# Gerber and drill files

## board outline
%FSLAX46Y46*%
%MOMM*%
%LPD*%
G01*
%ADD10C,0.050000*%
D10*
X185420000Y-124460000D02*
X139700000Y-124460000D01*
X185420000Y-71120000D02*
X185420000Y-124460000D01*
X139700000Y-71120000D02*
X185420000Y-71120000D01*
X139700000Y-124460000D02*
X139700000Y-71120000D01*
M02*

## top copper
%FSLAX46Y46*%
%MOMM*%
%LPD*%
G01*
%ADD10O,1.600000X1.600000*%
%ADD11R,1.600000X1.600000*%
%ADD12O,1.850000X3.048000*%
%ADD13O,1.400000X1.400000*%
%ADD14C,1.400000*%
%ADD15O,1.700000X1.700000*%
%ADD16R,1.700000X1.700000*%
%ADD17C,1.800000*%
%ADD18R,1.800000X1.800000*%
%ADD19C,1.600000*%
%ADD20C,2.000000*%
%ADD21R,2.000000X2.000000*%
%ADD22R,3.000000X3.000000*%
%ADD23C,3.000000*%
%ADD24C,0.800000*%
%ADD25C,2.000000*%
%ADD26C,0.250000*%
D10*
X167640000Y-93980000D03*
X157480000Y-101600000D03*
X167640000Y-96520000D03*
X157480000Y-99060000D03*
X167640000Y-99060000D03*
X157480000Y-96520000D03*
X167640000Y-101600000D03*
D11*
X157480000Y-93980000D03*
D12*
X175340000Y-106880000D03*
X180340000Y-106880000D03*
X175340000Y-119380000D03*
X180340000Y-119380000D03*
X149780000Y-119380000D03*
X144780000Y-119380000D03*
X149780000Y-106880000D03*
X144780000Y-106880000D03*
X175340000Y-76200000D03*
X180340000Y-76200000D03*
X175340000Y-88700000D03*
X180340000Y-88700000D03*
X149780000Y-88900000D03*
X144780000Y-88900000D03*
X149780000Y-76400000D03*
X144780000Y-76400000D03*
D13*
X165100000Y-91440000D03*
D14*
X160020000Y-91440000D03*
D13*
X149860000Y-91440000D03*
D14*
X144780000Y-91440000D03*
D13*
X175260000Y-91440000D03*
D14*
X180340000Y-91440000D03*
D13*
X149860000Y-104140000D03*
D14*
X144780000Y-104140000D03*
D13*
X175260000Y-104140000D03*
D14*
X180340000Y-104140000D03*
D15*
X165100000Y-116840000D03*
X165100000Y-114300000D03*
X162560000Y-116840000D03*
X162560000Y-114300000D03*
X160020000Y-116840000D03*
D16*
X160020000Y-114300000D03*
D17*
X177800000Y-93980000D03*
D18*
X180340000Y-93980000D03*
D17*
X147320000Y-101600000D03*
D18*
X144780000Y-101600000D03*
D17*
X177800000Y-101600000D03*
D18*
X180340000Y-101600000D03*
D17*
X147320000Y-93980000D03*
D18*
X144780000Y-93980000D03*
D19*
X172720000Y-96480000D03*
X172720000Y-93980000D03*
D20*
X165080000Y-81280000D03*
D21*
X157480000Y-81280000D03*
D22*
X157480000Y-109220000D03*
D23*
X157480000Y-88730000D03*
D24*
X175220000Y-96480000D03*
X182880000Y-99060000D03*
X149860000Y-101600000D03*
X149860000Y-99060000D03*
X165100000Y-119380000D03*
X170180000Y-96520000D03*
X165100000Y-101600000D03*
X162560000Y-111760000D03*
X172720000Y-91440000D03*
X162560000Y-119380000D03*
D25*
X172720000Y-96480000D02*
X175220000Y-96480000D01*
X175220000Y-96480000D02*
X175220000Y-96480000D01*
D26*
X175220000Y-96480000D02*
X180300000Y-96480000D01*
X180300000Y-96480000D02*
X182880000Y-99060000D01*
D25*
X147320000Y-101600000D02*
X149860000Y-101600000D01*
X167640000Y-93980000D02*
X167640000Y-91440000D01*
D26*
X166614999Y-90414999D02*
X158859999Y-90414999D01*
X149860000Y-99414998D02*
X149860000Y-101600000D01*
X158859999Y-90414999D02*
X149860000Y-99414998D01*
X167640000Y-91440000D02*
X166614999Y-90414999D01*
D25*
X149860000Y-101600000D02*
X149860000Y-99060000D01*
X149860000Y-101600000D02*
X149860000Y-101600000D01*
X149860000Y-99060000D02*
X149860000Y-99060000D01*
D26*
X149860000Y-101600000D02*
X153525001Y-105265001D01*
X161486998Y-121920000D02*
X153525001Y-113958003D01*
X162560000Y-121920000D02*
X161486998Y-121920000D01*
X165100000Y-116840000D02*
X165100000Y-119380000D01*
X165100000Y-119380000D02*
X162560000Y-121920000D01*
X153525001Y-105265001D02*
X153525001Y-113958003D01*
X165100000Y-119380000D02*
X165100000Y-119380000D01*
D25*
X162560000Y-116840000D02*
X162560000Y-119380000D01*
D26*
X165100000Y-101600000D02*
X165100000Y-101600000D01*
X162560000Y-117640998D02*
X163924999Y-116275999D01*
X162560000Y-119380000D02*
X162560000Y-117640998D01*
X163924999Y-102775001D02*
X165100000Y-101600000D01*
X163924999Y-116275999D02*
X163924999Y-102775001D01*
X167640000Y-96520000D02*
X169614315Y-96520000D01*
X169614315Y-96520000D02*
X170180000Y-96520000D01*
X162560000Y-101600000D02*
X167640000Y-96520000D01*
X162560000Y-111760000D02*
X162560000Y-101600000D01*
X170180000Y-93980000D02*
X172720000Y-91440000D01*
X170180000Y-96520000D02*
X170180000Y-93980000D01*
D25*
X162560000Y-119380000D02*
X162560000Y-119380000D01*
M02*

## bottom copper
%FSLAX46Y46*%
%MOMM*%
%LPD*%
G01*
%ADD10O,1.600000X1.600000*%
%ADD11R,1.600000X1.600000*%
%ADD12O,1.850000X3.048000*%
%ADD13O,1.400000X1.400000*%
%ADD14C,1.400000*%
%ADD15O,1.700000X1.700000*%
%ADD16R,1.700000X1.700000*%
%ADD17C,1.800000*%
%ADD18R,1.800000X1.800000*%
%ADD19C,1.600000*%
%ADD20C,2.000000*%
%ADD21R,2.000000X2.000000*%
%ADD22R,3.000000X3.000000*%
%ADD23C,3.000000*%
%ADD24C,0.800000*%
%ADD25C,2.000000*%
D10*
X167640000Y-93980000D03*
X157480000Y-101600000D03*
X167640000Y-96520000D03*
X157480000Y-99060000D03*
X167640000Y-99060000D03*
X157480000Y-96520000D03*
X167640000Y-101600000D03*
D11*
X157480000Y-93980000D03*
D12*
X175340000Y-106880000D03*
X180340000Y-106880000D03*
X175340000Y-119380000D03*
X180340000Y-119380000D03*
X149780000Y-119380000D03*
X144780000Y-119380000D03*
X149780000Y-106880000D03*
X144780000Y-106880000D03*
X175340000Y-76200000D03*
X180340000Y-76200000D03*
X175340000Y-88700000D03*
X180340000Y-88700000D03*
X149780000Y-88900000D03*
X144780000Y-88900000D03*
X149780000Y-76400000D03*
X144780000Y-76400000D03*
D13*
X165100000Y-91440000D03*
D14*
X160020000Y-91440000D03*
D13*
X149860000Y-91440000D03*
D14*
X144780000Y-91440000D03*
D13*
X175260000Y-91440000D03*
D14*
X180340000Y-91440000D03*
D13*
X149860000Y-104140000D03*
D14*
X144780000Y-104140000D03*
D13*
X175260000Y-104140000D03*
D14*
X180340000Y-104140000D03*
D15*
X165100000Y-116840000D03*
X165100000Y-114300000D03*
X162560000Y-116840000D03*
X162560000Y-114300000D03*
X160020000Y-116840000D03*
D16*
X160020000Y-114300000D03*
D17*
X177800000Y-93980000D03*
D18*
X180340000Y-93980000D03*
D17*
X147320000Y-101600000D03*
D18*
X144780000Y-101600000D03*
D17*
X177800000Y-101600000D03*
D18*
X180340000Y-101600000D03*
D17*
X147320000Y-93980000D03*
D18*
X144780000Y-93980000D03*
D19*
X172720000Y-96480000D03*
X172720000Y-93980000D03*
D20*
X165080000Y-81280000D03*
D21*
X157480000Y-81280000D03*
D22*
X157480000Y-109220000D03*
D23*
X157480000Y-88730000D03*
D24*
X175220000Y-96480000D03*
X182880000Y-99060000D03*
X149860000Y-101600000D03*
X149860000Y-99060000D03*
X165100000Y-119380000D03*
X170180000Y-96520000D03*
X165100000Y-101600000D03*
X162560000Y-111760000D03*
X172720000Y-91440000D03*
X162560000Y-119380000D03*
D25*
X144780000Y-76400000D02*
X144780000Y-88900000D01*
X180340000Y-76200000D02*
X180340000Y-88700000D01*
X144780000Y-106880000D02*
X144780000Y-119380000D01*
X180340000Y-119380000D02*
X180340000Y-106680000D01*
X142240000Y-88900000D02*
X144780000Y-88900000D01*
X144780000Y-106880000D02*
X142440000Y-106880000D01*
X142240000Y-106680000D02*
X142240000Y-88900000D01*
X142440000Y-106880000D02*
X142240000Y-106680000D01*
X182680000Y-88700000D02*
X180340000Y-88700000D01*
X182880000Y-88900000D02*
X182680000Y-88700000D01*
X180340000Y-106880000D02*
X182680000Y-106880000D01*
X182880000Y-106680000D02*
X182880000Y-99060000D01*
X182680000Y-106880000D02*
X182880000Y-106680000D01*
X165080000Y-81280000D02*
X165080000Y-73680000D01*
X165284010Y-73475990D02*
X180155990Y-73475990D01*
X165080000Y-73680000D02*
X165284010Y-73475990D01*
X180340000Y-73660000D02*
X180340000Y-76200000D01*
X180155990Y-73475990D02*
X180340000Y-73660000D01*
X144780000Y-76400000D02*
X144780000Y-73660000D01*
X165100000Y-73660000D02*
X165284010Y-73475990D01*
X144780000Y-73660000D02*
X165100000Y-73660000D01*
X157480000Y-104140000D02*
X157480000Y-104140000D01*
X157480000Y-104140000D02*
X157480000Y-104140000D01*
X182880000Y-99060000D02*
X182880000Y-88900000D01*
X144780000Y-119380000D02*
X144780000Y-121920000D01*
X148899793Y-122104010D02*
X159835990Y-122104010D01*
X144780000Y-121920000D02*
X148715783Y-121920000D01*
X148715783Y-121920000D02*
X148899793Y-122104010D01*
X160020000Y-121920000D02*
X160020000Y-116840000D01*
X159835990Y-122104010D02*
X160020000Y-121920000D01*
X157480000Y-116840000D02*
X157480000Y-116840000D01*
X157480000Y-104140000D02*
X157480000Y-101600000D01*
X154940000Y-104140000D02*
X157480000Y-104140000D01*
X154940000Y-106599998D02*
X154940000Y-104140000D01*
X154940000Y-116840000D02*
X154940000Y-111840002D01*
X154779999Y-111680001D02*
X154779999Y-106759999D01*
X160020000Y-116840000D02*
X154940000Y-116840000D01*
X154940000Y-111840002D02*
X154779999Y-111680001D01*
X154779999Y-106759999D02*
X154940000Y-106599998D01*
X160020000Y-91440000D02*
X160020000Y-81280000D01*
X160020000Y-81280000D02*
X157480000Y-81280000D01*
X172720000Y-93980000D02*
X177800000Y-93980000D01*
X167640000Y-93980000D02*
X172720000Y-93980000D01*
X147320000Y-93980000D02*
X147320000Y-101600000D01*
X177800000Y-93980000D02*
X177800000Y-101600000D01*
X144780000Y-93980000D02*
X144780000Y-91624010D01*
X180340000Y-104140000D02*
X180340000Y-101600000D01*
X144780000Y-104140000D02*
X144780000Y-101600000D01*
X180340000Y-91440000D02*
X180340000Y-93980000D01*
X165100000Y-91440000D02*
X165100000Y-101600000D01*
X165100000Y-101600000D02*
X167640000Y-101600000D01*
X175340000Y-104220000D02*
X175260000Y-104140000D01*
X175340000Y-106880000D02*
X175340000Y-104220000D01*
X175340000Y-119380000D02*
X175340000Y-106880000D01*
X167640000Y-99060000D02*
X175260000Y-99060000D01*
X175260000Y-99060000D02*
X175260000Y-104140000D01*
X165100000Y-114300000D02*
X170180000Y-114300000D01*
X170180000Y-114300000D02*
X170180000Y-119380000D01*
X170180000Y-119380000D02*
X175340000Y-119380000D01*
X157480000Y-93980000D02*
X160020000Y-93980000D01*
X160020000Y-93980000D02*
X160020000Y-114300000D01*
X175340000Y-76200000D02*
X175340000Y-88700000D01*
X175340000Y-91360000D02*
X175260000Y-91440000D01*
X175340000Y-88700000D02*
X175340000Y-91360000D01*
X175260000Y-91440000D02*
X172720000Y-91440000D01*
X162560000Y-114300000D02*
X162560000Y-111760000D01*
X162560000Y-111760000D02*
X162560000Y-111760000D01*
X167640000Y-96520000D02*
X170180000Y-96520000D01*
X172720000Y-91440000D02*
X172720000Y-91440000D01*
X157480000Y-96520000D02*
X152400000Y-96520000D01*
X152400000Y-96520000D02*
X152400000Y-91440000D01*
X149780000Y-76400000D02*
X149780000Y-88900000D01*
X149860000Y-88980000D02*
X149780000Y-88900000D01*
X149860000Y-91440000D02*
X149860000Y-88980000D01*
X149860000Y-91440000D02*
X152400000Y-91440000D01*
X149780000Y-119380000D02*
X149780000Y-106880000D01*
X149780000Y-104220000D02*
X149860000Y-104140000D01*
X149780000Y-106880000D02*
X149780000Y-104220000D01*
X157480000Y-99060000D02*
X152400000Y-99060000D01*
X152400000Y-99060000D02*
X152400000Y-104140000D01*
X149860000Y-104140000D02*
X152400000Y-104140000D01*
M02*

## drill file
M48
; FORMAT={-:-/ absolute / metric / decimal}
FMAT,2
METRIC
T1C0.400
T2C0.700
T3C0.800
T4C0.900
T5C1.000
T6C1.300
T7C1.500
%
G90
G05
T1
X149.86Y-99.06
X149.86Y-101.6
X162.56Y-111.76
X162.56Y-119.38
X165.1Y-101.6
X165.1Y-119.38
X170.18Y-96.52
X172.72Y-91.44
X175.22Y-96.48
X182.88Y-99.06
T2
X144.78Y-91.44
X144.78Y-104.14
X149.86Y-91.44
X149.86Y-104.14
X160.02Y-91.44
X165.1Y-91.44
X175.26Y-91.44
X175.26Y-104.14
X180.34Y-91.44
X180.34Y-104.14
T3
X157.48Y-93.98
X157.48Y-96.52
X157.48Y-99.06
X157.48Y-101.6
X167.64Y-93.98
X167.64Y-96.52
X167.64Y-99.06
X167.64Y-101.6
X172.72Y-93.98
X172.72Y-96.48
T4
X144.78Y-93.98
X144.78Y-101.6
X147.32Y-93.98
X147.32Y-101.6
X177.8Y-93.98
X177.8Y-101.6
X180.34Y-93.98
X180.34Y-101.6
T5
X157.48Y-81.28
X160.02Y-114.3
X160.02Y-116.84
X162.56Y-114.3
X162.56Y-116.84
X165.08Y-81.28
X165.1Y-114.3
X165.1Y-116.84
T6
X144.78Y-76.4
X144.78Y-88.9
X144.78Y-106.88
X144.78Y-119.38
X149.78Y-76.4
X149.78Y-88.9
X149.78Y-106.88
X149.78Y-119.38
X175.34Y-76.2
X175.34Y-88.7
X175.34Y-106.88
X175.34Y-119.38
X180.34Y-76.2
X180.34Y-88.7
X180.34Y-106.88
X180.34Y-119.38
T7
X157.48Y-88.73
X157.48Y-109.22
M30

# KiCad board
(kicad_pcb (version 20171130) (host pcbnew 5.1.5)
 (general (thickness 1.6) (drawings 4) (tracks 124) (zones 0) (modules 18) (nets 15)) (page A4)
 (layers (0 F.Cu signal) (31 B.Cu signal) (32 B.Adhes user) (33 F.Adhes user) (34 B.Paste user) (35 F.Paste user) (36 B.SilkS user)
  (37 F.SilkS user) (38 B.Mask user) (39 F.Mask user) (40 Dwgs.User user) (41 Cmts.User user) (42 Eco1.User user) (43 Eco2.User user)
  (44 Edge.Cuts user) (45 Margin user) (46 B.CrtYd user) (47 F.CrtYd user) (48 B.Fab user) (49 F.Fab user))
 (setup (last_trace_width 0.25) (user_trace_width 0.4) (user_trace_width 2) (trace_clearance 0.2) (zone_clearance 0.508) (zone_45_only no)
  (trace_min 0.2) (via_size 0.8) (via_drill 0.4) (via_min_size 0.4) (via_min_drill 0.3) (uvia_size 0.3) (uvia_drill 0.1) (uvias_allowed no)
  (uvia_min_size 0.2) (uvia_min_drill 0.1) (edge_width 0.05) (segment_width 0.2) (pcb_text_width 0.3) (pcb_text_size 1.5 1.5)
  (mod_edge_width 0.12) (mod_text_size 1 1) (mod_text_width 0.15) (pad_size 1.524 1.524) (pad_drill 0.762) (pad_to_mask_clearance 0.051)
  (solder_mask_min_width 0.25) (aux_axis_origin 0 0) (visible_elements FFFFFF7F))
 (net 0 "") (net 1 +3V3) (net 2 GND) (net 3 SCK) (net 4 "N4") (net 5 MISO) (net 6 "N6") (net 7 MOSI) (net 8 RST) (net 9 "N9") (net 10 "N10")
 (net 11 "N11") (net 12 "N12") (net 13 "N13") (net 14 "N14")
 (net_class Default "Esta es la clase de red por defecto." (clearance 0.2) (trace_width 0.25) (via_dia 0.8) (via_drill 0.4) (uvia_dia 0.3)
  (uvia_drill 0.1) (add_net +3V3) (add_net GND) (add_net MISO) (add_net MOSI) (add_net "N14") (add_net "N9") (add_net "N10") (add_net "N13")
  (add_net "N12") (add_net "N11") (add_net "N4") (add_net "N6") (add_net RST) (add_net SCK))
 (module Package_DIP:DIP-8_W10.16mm (layer F.Cu) (at 157.48 93.98)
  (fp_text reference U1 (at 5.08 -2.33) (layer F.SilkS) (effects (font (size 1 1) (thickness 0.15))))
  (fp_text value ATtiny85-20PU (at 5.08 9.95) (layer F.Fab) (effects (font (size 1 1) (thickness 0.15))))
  (pad 8 thru_hole oval (at 10.16 0) (size 1.6 1.6) (drill 0.8) (layers *.Cu *.Mask) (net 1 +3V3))
  (pad 4 thru_hole oval (at 0 7.62) (size 1.6 1.6) (drill 0.8) (layers *.Cu *.Mask) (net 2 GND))
  (pad 7 thru_hole oval (at 10.16 2.54) (size 1.6 1.6) (drill 0.8) (layers *.Cu *.Mask) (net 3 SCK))
  (pad 3 thru_hole oval (at 0 5.08) (size 1.6 1.6) (drill 0.8) (layers *.Cu *.Mask) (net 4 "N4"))
  (pad 6 thru_hole oval (at 10.16 5.08) (size 1.6 1.6) (drill 0.8) (layers *.Cu *.Mask) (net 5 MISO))
  (pad 2 thru_hole oval (at 0 2.54) (size 1.6 1.6) (drill 0.8) (layers *.Cu *.Mask) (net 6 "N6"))
  (pad 5 thru_hole oval (at 10.16 7.62) (size 1.6 1.6) (drill 0.8) (layers *.Cu *.Mask) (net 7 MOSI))
  (pad 1 thru_hole rect (at 0 0) (size 1.6 1.6) (drill 0.8) (layers *.Cu *.Mask) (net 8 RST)))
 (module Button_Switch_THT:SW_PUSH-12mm (layer F.Cu) (at 180.34 106.88 270)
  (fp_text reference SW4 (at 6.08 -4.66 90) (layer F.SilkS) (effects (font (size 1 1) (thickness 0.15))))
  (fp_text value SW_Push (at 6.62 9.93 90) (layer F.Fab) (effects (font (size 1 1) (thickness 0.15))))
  (pad 2 thru_hole oval (at 0 5 270) (size 3.048 1.85) (drill 1.3) (layers *.Cu *.Mask) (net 5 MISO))
  (pad 1 thru_hole oval (at 0 0 270) (size 3.048 1.85) (drill 1.3) (layers *.Cu *.Mask) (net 2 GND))
  (pad 2 thru_hole oval (at 12.5 5 270) (size 3.048 1.85) (drill 1.3) (layers *.Cu *.Mask) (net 5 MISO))
  (pad 1 thru_hole oval (at 12.5 0 270) (size 3.048 1.85) (drill 1.3) (layers *.Cu *.Mask) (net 2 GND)))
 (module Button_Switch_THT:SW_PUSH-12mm (layer F.Cu) (at 144.78 119.38 90)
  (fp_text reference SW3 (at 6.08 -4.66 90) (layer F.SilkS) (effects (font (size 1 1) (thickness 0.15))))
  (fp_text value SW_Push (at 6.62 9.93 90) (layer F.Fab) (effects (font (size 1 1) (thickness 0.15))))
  (pad 2 thru_hole oval (at 0 5 90) (size 3.048 1.85) (drill 1.3) (layers *.Cu *.Mask) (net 4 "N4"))
  (pad 1 thru_hole oval (at 0 0 90) (size 3.048 1.85) (drill 1.3) (layers *.Cu *.Mask) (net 2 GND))
  (pad 2 thru_hole oval (at 12.5 5 90) (size 3.048 1.85) (drill 1.3) (layers *.Cu *.Mask) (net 4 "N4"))
  (pad 1 thru_hole oval (at 12.5 0 90) (size 3.048 1.85) (drill 1.3) (layers *.Cu *.Mask) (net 2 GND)))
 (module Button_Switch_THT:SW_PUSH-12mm (layer F.Cu) (at 180.34 76.2 270)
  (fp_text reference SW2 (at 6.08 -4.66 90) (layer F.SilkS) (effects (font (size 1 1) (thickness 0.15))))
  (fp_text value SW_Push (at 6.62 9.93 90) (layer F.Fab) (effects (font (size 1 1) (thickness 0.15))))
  (pad 2 thru_hole oval (at 0 5 270) (size 3.048 1.85) (drill 1.3) (layers *.Cu *.Mask) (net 3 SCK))
  (pad 1 thru_hole oval (at 0 0 270) (size 3.048 1.85) (drill 1.3) (layers *.Cu *.Mask) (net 2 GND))
  (pad 2 thru_hole oval (at 12.5 5 270) (size 3.048 1.85) (drill 1.3) (layers *.Cu *.Mask) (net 3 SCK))
  (pad 1 thru_hole oval (at 12.5 0 270) (size 3.048 1.85) (drill 1.3) (layers *.Cu *.Mask) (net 2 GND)))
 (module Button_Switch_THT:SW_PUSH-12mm (layer F.Cu) (at 144.78 88.9 90)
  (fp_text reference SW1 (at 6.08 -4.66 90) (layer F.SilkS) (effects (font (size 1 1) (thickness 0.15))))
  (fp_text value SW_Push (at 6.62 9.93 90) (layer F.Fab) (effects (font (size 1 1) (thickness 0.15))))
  (pad 2 thru_hole oval (at 0 5 90) (size 3.048 1.85) (drill 1.3) (layers *.Cu *.Mask) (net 6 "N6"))
  (pad 1 thru_hole oval (at 0 0 90) (size 3.048 1.85) (drill 1.3) (layers *.Cu *.Mask) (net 2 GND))
  (pad 2 thru_hole oval (at 12.5 5 90) (size 3.048 1.85) (drill 1.3) (layers *.Cu *.Mask) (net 6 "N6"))
  (pad 1 thru_hole oval (at 12.5 0 90) (size 3.048 1.85) (drill 1.3) (layers *.Cu *.Mask) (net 2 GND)))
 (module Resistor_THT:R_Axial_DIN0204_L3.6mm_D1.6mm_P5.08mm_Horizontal (layer F.Cu) (at 160.02 91.44)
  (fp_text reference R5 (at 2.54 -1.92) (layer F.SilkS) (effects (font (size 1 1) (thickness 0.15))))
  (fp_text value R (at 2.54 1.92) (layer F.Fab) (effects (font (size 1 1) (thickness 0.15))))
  (pad 2 thru_hole oval (at 5.08 0) (size 1.4 1.4) (drill 0.7) (layers *.Cu *.Mask) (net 7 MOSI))
  (pad 1 thru_hole circle (at 0 0) (size 1.4 1.4) (drill 0.7) (layers *.Cu *.Mask) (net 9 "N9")))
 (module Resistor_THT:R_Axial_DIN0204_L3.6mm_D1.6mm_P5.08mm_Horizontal (layer F.Cu) (at 144.78 91.44)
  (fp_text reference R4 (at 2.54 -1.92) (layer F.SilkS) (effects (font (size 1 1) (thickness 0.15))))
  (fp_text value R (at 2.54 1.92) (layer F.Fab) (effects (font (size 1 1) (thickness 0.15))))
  (pad 2 thru_hole oval (at 5.08 0) (size 1.4 1.4) (drill 0.7) (layers *.Cu *.Mask) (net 6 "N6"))
  (pad 1 thru_hole circle (at 0 0) (size 1.4 1.4) (drill 0.7) (layers *.Cu *.Mask) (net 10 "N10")))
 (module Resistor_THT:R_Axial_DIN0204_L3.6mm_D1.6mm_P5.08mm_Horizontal (layer F.Cu) (at 180.34 91.44 180)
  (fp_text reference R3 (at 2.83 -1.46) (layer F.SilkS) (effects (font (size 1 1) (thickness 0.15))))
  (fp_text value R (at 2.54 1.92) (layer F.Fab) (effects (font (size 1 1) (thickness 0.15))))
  (pad 2 thru_hole oval (at 5.08 0 180) (size 1.4 1.4) (drill 0.7) (layers *.Cu *.Mask) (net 3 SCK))
  (pad 1 thru_hole circle (at 0 0 180) (size 1.4 1.4) (drill 0.7) (layers *.Cu *.Mask) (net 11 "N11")))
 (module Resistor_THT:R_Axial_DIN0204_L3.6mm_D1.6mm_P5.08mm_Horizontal (layer F.Cu) (at 144.78 104.14)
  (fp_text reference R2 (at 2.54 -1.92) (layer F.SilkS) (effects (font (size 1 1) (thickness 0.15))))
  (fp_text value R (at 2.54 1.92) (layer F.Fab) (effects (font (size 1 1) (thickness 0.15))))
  (pad 2 thru_hole oval (at 5.08 0) (size 1.4 1.4) (drill 0.7) (layers *.Cu *.Mask) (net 4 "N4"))
  (pad 1 thru_hole circle (at 0 0) (size 1.4 1.4) (drill 0.7) (layers *.Cu *.Mask) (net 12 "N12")))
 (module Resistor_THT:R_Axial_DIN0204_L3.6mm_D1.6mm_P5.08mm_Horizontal (layer F.Cu) (at 180.34 104.14 180)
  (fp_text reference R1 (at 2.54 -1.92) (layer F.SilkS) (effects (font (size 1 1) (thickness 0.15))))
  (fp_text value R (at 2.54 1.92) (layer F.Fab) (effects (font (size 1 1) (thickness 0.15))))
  (pad 2 thru_hole oval (at 5.08 0 180) (size 1.4 1.4) (drill 0.7) (layers *.Cu *.Mask) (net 5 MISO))
  (pad 1 thru_hole circle (at 0 0 180) (size 1.4 1.4) (drill 0.7) (layers *.Cu *.Mask) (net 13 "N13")))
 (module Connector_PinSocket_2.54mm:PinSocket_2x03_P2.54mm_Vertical (layer F.Cu) (at 160.02 114.3 90)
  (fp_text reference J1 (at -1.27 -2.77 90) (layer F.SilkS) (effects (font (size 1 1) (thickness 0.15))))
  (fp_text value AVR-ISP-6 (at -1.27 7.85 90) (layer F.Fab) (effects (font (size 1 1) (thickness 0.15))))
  (pad 6 thru_hole oval (at -2.54 5.08 90) (size 1.7 1.7) (drill 1) (layers *.Cu *.Mask) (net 1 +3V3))
  (pad 5 thru_hole oval (at 0 5.08 90) (size 1.7 1.7) (drill 1) (layers *.Cu *.Mask) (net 5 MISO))
  (pad 4 thru_hole oval (at -2.54 2.54 90) (size 1.7 1.7) (drill 1) (layers *.Cu *.Mask) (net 7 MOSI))
  (pad 3 thru_hole oval (at 0 2.54 90) (size 1.7 1.7) (drill 1) (layers *.Cu *.Mask) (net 3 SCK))
  (pad 2 thru_hole oval (at -2.54 0 90) (size 1.7 1.7) (drill 1) (layers *.Cu *.Mask) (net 2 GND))
  (pad 1 thru_hole rect (at 0 0 90) (size 1.7 1.7) (drill 1) (layers *.Cu *.Mask) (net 8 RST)))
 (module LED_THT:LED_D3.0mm (layer F.Cu) (at 180.34 93.98 180)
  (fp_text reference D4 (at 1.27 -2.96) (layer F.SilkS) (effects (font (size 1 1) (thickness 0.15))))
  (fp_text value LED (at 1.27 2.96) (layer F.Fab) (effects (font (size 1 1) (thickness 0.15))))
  (pad 2 thru_hole circle (at 2.54 0 180) (size 1.8 1.8) (drill 0.9) (layers *.Cu *.Mask) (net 1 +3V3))
  (pad 1 thru_hole rect (at 0 0 180) (size 1.8 1.8) (drill 0.9) (layers *.Cu *.Mask) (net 11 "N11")))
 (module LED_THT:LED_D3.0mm (layer F.Cu) (at 144.78 101.6)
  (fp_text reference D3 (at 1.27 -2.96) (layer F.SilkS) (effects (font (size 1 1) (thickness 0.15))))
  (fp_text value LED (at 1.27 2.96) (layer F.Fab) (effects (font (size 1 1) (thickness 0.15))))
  (pad 2 thru_hole circle (at 2.54 0) (size 1.8 1.8) (drill 0.9) (layers *.Cu *.Mask) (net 1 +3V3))
  (pad 1 thru_hole rect (at 0 0) (size 1.8 1.8) (drill 0.9) (layers *.Cu *.Mask) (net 12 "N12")))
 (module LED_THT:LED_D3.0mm (layer F.Cu) (at 180.34 101.6 180)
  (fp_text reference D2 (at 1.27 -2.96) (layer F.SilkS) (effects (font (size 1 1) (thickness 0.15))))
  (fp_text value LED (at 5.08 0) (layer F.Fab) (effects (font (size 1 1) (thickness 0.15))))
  (pad 2 thru_hole circle (at 2.54 0 180) (size 1.8 1.8) (drill 0.9) (layers *.Cu *.Mask) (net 1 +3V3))
  (pad 1 thru_hole rect (at 0 0 180) (size 1.8 1.8) (drill 0.9) (layers *.Cu *.Mask) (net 13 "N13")))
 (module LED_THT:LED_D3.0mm (layer F.Cu) (at 144.78 93.98)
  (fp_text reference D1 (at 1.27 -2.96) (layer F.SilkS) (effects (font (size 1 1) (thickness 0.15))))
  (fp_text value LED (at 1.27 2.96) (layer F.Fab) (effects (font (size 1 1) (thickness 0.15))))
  (pad 2 thru_hole circle (at 2.54 0) (size 1.8 1.8) (drill 0.9) (layers *.Cu *.Mask) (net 1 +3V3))
  (pad 1 thru_hole rect (at 0 0) (size 1.8 1.8) (drill 0.9) (layers *.Cu *.Mask) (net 10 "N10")))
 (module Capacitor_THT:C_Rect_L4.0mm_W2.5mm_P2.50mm (layer F.Cu) (at 172.72 93.98 270)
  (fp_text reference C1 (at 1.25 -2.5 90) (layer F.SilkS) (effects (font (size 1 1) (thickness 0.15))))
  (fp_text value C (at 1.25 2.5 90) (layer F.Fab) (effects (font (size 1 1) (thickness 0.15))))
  (pad 2 thru_hole circle (at 2.5 0 270) (size 1.6 1.6) (drill 0.8) (layers *.Cu *.Mask) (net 2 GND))
  (pad 1 thru_hole circle (at 0 0 270) (size 1.6 1.6) (drill 0.8) (layers *.Cu *.Mask) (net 1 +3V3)))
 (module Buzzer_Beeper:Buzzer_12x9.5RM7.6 (layer F.Cu) (at 157.48 81.28)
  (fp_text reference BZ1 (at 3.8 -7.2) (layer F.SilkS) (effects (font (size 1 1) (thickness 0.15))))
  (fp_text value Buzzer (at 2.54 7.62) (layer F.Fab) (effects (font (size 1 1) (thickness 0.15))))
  (pad 2 thru_hole circle (at 7.6 0) (size 2 2) (drill 1) (layers *.Cu *.Mask) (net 2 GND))
  (pad 1 thru_hole rect (at 0 0) (size 2 2) (drill 1) (layers *.Cu *.Mask) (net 9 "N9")))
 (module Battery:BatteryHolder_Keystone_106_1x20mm (layer B.Cu) (at 157.48 109.22 90)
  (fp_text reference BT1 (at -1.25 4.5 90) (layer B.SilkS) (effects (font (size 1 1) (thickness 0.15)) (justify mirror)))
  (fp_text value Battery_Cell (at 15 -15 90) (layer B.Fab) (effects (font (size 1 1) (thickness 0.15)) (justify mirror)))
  (pad 1 thru_hole rect (at 0 0 90) (size 3 3) (drill 1.5) (layers *.Cu *.Mask) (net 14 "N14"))
  (pad 2 thru_hole circle (at 20.49 0 90) (size 3 3) (drill 1.5) (layers *.Cu *.Mask) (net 2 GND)))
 (gr_line (start 185.42 124.46) (end 139.7 124.46) (layer Edge.Cuts) (width 0.05))
 (gr_line (start 185.42 71.12) (end 185.42 124.46) (layer Edge.Cuts) (width 0.05))
 (gr_line (start 139.7 71.12) (end 185.42 71.12) (layer Edge.Cuts) (width 0.05))
 (gr_line (start 139.7 124.46) (end 139.7 71.12) (layer Edge.Cuts) (width 0.05))
 (segment (start 144.78 76.4) (end 144.78 88.9) (width 2) (layer B.Cu) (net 2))
 (segment (start 180.34 76.2) (end 180.34 88.7) (width 2) (layer B.Cu) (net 2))
 (segment (start 144.78 106.88) (end 144.78 119.38) (width 2) (layer B.Cu) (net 2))
 (segment (start 180.34 119.38) (end 180.34 106.68) (width 2) (layer B.Cu) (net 2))
 (segment (start 142.24 88.9) (end 144.78 88.9) (width 2) (layer B.Cu) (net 2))
 (segment (start 144.78 106.88) (end 142.44 106.88) (width 2) (layer B.Cu) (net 2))
 (segment (start 142.24 106.68) (end 142.24 88.9) (width 2) (layer B.Cu) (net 2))
 (segment (start 142.44 106.88) (end 142.24 106.68) (width 2) (layer B.Cu) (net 2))
 (segment (start 182.68 88.7) (end 180.34 88.7) (width 2) (layer B.Cu) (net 2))
 (segment (start 182.88 88.9) (end 182.68 88.7) (width 2) (layer B.Cu) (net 2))
 (segment (start 180.34 106.88) (end 182.68 106.88) (width 2) (layer B.Cu) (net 2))
 (segment (start 182.88 106.68) (end 182.88 99.06) (width 2) (layer B.Cu) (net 2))
 (segment (start 182.68 106.88) (end 182.88 106.68) (width 2) (layer B.Cu) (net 2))
 (segment (start 165.08 81.28) (end 165.08 73.68) (width 2) (layer B.Cu) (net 2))
 (segment (start 165.28401 73.47599) (end 180.15599 73.47599) (width 2) (layer B.Cu) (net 2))
 (segment (start 165.08 73.68) (end 165.28401 73.47599) (width 2) (layer B.Cu) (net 2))
 (segment (start 180.34 73.66) (end 180.34 76.2) (width 2) (layer B.Cu) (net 2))
 (segment (start 180.15599 73.47599) (end 180.34 73.66) (width 2) (layer B.Cu) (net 2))
 (segment (start 144.78 76.4) (end 144.78 73.66) (width 2) (layer B.Cu) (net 2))
 (segment (start 165.1 73.66) (end 165.28401 73.47599) (width 2) (layer B.Cu) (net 2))
 (segment (start 144.78 73.66) (end 165.1 73.66) (width 2) (layer B.Cu) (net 2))
 (segment (start 172.72 96.48) (end 175.22 96.48) (width 2) (layer F.Cu) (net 2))
 (segment (start 157.48 104.14) (end 157.48 104.14) (width 2) (layer B.Cu) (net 2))
 (segment (start 157.48 104.14) (end 157.48 104.14) (width 2) (layer B.Cu) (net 2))
 (segment (start 175.22 96.48) (end 175.22 96.48) (width 2) (layer F.Cu) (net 2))
 (via (at 175.22 96.48) (size 0.8) (drill 0.4) (layers F.Cu B.Cu) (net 2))
 (segment (start 175.22 96.48) (end 180.3 96.48) (width 0.25) (layer F.Cu) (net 2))
 (segment (start 182.88 99.06) (end 182.88 88.9) (width 2) (layer B.Cu) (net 2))
 (via (at 182.88 99.06) (size 0.8) (drill 0.4) (layers F.Cu B.Cu) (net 2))
 (segment (start 180.3 96.48) (end 182.88 99.06) (width 0.25) (layer F.Cu) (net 2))
 (segment (start 144.78 119.38) (end 144.78 121.92) (width 2) (layer B.Cu) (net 2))
 (segment (start 148.899793 122.10401) (end 159.83599 122.10401) (width 2) (layer B.Cu) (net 2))
 (segment (start 144.78 121.92) (end 148.715783 121.92) (width 2) (layer B.Cu) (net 2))
 (segment (start 148.715783 121.92) (end 148.899793 122.10401) (width 2) (layer B.Cu) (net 2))
 (segment (start 160.02 121.92) (end 160.02 116.84) (width 2) (layer B.Cu) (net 2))
 (segment (start 159.83599 122.10401) (end 160.02 121.92) (width 2) (layer B.Cu) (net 2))
 (segment (start 157.48 116.84) (end 157.48 116.84) (width 2) (layer B.Cu) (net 2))
 (segment (start 157.48 104.14) (end 157.48 101.6) (width 2) (layer B.Cu) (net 2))
 (segment (start 154.94 104.14) (end 157.48 104.14) (width 2) (layer B.Cu) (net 2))
 (segment (start 154.94 106.599998) (end 154.94 104.14) (width 2) (layer B.Cu) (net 2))
 (segment (start 154.94 116.84) (end 154.94 111.840002) (width 2) (layer B.Cu) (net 2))
 (segment (start 154.779999 111.680001) (end 154.779999 106.759999) (width 2) (layer B.Cu) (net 2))
 (segment (start 160.02 116.84) (end 154.94 116.84) (width 2) (layer B.Cu) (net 2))
 (segment (start 154.94 111.840002) (end 154.779999 111.680001) (width 2) (layer B.Cu) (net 2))
 (segment (start 154.779999 106.759999) (end 154.94 106.599998) (width 2) (layer B.Cu) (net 2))
 (segment (start 160.02 91.44) (end 160.02 81.28) (width 2) (layer B.Cu) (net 9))
 (segment (start 160.02 81.28) (end 157.48 81.28) (width 2) (layer B.Cu) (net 9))
 (segment (start 172.72 93.98) (end 177.8 93.98) (width 2) (layer B.Cu) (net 1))
 (segment (start 167.64 93.98) (end 172.72 93.98) (width 2) (layer B.Cu) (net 1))
 (segment (start 147.32 93.98) (end 147.32 101.6) (width 2) (layer B.Cu) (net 1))
 (segment (start 177.8 93.98) (end 177.8 101.6) (width 2) (layer B.Cu) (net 1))
 (segment (start 147.32 101.6) (end 149.86 101.6) (width 2) (layer F.Cu) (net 1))
 (segment (start 167.64 93.98) (end 167.64 91.44) (width 2) (layer F.Cu) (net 1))
 (segment (start 166.614999 90.414999) (end 158.859999 90.414999) (width 0.25) (layer F.Cu) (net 1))
 (segment (start 149.86 99.414998) (end 149.86 101.6) (width 0.25) (layer F.Cu) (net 1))
 (segment (start 158.859999 90.414999) (end 149.86 99.414998) (width 0.25) (layer F.Cu) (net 1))
 (segment (start 167.64 91.44) (end 166.614999 90.414999) (width 0.25) (layer F.Cu) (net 1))
 (segment (start 149.86 101.6) (end 149.86 99.06) (width 2) (layer F.Cu) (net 1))
 (segment (start 149.86 101.6) (end 149.86 101.6) (width 2) (layer F.Cu) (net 1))
 (via (at 149.86 101.6) (size 0.8) (drill 0.4) (layers F.Cu B.Cu) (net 1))
 (segment (start 149.86 99.06) (end 149.86 99.06) (width 2) (layer F.Cu) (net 1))
 (via (at 149.86 99.06) (size 0.8) (drill 0.4) (layers F.Cu B.Cu) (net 1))
 (segment (start 149.86 101.6) (end 153.525001 105.265001) (width 0.25) (layer F.Cu) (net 1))
 (segment (start 161.486998 121.92) (end 153.525001 113.958003) (width 0.25) (layer F.Cu) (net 1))
 (segment (start 162.56 121.92) (end 161.486998 121.92) (width 0.25) (layer F.Cu) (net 1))
 (segment (start 165.1 116.84) (end 165.1 119.38) (width 0.25) (layer F.Cu) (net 1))
 (segment (start 165.1 119.38) (end 162.56 121.92) (width 0.25) (layer F.Cu) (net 1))
 (segment (start 153.525001 105.265001) (end 153.525001 113.958003) (width 0.25) (layer F.Cu) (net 1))
 (segment (start 165.1 119.38) (end 165.1 119.38) (width 0.25) (layer F.Cu) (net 1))
 (via (at 165.1 119.38) (size 0.8) (drill 0.4) (layers F.Cu B.Cu) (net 1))
 (segment (start 144.78 93.98) (end 144.78 91.62401) (width 2) (layer B.Cu) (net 10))
 (segment (start 180.34 104.14) (end 180.34 101.6) (width 2) (layer B.Cu) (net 13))
 (segment (start 144.78 104.14) (end 144.78 101.6) (width 2) (layer B.Cu) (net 12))
 (segment (start 180.34 91.44) (end 180.34 93.98) (width 2) (layer B.Cu) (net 11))
 (via (at 170.18 96.52) (size 0.8) (drill 0.4) (layers F.Cu B.Cu) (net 3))
 (segment (start 165.1 91.44) (end 165.1 101.6) (width 2) (layer B.Cu) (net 7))
 (segment (start 165.1 101.6) (end 167.64 101.6) (width 2) (layer B.Cu) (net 7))
 (segment (start 162.56 116.84) (end 162.56 119.38) (width 2) (layer F.Cu) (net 7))
 (segment (start 165.1 101.6) (end 165.1 101.6) (width 0.25) (layer F.Cu) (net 7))
 (via (at 165.1 101.6) (size 0.8) (drill 0.4) (layers F.Cu B.Cu) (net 7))
 (segment (start 162.56 117.640998) (end 163.924999 116.275999) (width 0.25) (layer F.Cu) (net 7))
 (segment (start 162.56 119.38) (end 162.56 117.640998) (width 0.25) (layer F.Cu) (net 7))
 (segment (start 163.924999 102.775001) (end 165.1 101.6) (width 0.25) (layer F.Cu) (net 7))
 (segment (start 163.924999 116.275999) (end 163.924999 102.775001) (width 0.25) (layer F.Cu) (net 7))
 (segment (start 175.34 104.22) (end 175.26 104.14) (width 2) (layer B.Cu) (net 5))
 (segment (start 175.34 106.88) (end 175.34 104.22) (width 2) (layer B.Cu) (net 5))
 (segment (start 175.34 119.38) (end 175.34 106.88) (width 2) (layer B.Cu) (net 5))
 (segment (start 167.64 99.06) (end 175.26 99.06) (width 2) (layer B.Cu) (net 5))
 (segment (start 175.26 99.06) (end 175.26 104.14) (width 2) (layer B.Cu) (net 5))
 (segment (start 165.1 114.3) (end 170.18 114.3) (width 2) (layer B.Cu) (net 5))
 (segment (start 170.18 114.3) (end 170.18 119.38) (width 2) (layer B.Cu) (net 5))
 (segment (start 170.18 119.38) (end 175.34 119.38) (width 2) (layer B.Cu) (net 5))
 (segment (start 157.48 93.98) (end 160.02 93.98) (width 2) (layer B.Cu) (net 8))
 (segment (start 160.02 93.98) (end 160.02 114.3) (width 2) (layer B.Cu) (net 8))
 (segment (start 175.34 76.2) (end 175.34 88.7) (width 2) (layer B.Cu) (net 3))
 (segment (start 175.34 91.36) (end 175.26 91.44) (width 2) (layer B.Cu) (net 3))
 (segment (start 175.34 88.7) (end 175.34 91.36) (width 2) (layer B.Cu) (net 3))
 (segment (start 175.26 91.44) (end 172.72 91.44) (width 2) (layer B.Cu) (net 3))
 (segment (start 162.56 114.3) (end 162.56 111.76) (width 2) (layer B.Cu) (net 3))
 (segment (start 162.56 111.76) (end 162.56 111.76) (width 2) (layer B.Cu) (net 3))
 (via (at 162.56 111.76) (size 0.8) (drill 0.4) (layers F.Cu B.Cu) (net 3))
 (segment (start 167.64 96.52) (end 169.614315 96.52) (width 0.25) (layer F.Cu) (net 3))
 (segment (start 169.614315 96.52) (end 170.18 96.52) (width 0.25) (layer F.Cu) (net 3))
 (segment (start 162.56 101.6) (end 167.64 96.52) (width 0.25) (layer F.Cu) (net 3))
 (segment (start 162.56 111.76) (end 162.56 101.6) (width 0.25) (layer F.Cu) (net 3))
 (segment (start 167.64 96.52) (end 170.18 96.52) (width 2) (layer B.Cu) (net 3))
 (segment (start 172.72 91.44) (end 172.72 91.44) (width 2) (layer B.Cu) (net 3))
 (via (at 172.72 91.44) (size 0.8) (drill 0.4) (layers F.Cu B.Cu) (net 3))
 (segment (start 170.18 93.98) (end 172.72 91.44) (width 0.25) (layer F.Cu) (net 3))
 (segment (start 170.18 96.52) (end 170.18 93.98) (width 0.25) (layer F.Cu) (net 3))
 (segment (start 162.56 119.38) (end 162.56 119.38) (width 2) (layer F.Cu) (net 7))
 (via (at 162.56 119.38) (size 0.8) (drill 0.4) (layers F.Cu B.Cu) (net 7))
 (segment (start 157.48 96.52) (end 152.4 96.52) (width 2) (layer B.Cu) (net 6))
 (segment (start 152.4 96.52) (end 152.4 91.44) (width 2) (layer B.Cu) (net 6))
 (segment (start 149.78 76.4) (end 149.78 88.9) (width 2) (layer B.Cu) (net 6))
 (segment (start 149.86 88.98) (end 149.78 88.9) (width 2) (layer B.Cu) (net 6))
 (segment (start 149.86 91.44) (end 149.86 88.98) (width 2) (layer B.Cu) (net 6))
 (segment (start 149.86 91.44) (end 152.4 91.44) (width 2) (layer B.Cu) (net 6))
 (segment (start 149.78 119.38) (end 149.78 106.88) (width 2) (layer B.Cu) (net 4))
 (segment (start 149.78 104.22) (end 149.86 104.14) (width 2) (layer B.Cu) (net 4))
 (segment (start 149.78 106.88) (end 149.78 104.22) (width 2) (layer B.Cu) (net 4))
 (segment (start 157.48 99.06) (end 152.4 99.06) (width 2) (layer B.Cu) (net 4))
 (segment (start 152.4 99.06) (end 152.4 104.14) (width 2) (layer B.Cu) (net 4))
 (segment (start 149.86 104.14) (end 152.4 104.14) (width 2) (layer B.Cu) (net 4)))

